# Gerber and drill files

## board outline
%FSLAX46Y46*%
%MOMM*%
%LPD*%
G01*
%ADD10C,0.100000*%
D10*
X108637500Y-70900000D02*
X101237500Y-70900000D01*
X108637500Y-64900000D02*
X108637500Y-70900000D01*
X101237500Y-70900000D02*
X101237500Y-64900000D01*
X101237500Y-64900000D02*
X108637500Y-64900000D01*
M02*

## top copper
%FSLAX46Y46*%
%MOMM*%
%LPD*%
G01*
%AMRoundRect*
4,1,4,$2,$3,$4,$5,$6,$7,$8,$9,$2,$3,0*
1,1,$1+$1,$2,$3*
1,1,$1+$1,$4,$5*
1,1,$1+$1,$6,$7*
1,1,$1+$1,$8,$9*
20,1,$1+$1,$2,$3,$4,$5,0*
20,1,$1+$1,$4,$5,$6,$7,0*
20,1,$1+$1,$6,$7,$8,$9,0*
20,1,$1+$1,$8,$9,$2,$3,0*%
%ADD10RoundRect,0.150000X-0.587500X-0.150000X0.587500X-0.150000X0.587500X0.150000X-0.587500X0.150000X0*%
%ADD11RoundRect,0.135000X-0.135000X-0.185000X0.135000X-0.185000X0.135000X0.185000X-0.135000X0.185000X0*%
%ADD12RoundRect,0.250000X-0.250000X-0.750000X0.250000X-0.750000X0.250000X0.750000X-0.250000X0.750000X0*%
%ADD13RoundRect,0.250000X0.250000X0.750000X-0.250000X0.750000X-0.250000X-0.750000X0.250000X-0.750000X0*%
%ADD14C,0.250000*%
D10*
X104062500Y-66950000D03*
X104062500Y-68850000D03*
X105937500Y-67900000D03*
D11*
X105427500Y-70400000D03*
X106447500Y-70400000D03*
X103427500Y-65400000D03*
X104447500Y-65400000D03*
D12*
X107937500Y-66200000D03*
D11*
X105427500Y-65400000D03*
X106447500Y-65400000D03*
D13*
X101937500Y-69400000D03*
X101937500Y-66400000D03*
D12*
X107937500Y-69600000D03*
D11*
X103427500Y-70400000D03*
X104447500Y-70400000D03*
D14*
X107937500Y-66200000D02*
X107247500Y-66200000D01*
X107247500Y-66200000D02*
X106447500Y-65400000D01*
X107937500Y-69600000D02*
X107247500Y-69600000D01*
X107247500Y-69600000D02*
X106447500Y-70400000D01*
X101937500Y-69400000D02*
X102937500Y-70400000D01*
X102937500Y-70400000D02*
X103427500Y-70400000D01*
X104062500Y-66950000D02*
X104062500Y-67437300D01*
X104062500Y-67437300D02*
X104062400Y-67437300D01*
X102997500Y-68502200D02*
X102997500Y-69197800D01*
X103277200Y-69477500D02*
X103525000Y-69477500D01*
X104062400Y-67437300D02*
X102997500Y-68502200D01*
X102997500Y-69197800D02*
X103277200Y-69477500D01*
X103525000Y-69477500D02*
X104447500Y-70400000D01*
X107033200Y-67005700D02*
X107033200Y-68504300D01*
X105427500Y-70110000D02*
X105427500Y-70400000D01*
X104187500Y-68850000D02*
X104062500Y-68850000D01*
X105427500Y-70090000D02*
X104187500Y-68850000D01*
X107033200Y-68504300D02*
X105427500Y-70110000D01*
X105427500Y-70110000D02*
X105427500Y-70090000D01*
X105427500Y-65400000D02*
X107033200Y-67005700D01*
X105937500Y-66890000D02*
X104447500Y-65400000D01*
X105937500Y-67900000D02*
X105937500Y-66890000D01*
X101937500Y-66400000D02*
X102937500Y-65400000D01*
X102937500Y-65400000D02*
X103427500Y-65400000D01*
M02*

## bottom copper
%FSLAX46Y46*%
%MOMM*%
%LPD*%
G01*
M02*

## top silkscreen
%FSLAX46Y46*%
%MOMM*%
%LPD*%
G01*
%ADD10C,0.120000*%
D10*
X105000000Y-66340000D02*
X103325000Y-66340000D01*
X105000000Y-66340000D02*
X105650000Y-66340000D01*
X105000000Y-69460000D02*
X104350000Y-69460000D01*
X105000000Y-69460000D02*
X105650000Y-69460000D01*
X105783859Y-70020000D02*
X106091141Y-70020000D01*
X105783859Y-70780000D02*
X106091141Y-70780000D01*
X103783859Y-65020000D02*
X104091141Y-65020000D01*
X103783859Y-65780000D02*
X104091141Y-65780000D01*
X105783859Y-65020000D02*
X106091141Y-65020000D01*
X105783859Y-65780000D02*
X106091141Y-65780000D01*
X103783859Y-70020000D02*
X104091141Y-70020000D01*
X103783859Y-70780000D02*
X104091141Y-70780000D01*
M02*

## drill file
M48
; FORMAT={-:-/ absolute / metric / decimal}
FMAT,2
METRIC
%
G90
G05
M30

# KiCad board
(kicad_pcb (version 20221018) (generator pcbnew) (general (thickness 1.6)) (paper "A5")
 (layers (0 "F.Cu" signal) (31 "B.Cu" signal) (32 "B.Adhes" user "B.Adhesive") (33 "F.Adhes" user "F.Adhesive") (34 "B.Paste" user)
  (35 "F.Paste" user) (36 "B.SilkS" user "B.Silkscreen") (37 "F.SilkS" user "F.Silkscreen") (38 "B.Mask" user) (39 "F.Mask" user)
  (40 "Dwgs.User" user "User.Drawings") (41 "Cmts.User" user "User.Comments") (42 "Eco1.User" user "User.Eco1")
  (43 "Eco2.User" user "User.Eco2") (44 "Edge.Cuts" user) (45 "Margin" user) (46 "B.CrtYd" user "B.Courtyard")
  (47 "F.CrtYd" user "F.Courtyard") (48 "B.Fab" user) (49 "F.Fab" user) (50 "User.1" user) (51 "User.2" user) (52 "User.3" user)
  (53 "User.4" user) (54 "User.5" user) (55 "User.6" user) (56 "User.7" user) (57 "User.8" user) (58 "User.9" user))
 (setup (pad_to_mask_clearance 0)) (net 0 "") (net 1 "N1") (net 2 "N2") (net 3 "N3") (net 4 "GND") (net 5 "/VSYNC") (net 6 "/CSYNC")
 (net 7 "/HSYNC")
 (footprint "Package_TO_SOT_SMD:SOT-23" (layer "F.Cu") (at 105 67.9)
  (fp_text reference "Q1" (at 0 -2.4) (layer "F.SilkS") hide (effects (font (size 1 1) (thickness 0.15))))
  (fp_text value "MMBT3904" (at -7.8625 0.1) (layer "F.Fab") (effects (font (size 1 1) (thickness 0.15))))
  (fp_line (start 0 -1.56) (end -1.675 -1.56) (stroke (width 0.12) (type solid)) (layer "F.SilkS"))
  (fp_line (start 0 -1.56) (end 0.65 -1.56) (stroke (width 0.12) (type solid)) (layer "F.SilkS"))
  (fp_line (start 0 1.56) (end -0.65 1.56) (stroke (width 0.12) (type solid)) (layer "F.SilkS"))
  (fp_line (start 0 1.56) (end 0.65 1.56) (stroke (width 0.12) (type solid)) (layer "F.SilkS"))
  (pad "1" smd roundrect (at -0.9375 -0.95) (size 1.475 0.6) (layers "F.Cu" "F.Paste" "F.Mask") (roundrect_rratio 0.25) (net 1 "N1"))
  (pad "2" smd roundrect (at -0.9375 0.95) (size 1.475 0.6) (layers "F.Cu" "F.Paste" "F.Mask") (roundrect_rratio 0.25) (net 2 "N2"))
  (pad "3" smd roundrect (at 0.9375 0) (size 1.475 0.6) (layers "F.Cu" "F.Paste" "F.Mask") (roundrect_rratio 0.25) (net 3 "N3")))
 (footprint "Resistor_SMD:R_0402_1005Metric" (layer "F.Cu") (at 105.9375 70.4)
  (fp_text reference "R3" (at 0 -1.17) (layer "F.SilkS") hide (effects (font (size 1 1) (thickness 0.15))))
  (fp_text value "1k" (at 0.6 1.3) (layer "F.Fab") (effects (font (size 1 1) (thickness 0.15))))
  (fp_line (start -0.153641 -0.38) (end 0.153641 -0.38) (stroke (width 0.12) (type solid)) (layer "F.SilkS"))
  (fp_line (start -0.153641 0.38) (end 0.153641 0.38) (stroke (width 0.12) (type solid)) (layer "F.SilkS"))
  (pad "1" smd roundrect (at -0.51 0) (size 0.54 0.64) (layers "F.Cu" "F.Paste" "F.Mask") (roundrect_rratio 0.25) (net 2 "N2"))
  (pad "2" smd roundrect (at 0.51 0) (size 0.54 0.64) (layers "F.Cu" "F.Paste" "F.Mask") (roundrect_rratio 0.25) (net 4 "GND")))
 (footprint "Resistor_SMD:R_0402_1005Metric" (layer "F.Cu") (at 103.9375 65.4)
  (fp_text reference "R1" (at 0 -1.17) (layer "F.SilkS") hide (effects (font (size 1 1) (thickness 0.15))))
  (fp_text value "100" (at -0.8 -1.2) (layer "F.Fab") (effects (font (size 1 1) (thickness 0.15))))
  (fp_line (start -0.153641 -0.38) (end 0.153641 -0.38) (stroke (width 0.12) (type solid)) (layer "F.SilkS"))
  (fp_line (start -0.153641 0.38) (end 0.153641 0.38) (stroke (width 0.12) (type solid)) (layer "F.SilkS"))
  (pad "1" smd roundrect (at -0.51 0) (size 0.54 0.64) (layers "F.Cu" "F.Paste" "F.Mask") (roundrect_rratio 0.25) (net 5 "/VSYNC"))
  (pad "2" smd roundrect (at 0.51 0) (size 0.54 0.64) (layers "F.Cu" "F.Paste" "F.Mask") (roundrect_rratio 0.25) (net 3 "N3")))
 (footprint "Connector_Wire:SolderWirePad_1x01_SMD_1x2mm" (layer "F.Cu") (at 107.9375 66.2)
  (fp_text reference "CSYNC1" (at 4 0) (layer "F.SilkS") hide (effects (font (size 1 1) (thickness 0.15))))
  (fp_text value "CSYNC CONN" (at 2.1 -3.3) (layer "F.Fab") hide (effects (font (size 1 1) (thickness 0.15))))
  (pad "1" smd roundrect (at 0 0) (size 1 2) (layers "F.Cu" "F.Paste" "F.Mask") (roundrect_rratio 0.25) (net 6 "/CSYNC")))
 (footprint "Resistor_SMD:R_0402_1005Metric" (layer "F.Cu") (at 105.9375 65.4)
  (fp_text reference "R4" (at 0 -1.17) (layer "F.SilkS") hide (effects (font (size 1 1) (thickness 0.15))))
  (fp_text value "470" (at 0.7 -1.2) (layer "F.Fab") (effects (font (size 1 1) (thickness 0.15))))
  (fp_line (start -0.153641 -0.38) (end 0.153641 -0.38) (stroke (width 0.12) (type solid)) (layer "F.SilkS"))
  (fp_line (start -0.153641 0.38) (end 0.153641 0.38) (stroke (width 0.12) (type solid)) (layer "F.SilkS"))
  (pad "1" smd roundrect (at -0.51 0) (size 0.54 0.64) (layers "F.Cu" "F.Paste" "F.Mask") (roundrect_rratio 0.25) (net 2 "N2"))
  (pad "2" smd roundrect (at 0.51 0) (size 0.54 0.64) (layers "F.Cu" "F.Paste" "F.Mask") (roundrect_rratio 0.25) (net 6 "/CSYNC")))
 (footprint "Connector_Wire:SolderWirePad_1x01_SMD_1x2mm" (layer "F.Cu") (at 101.9375 69.4 180)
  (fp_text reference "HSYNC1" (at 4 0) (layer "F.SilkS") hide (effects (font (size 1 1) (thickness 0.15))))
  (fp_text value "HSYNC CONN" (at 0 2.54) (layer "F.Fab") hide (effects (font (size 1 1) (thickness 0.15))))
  (pad "1" smd roundrect (at 0 0 180) (size 1 2) (layers "F.Cu" "F.Paste" "F.Mask") (roundrect_rratio 0.25) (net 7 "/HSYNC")))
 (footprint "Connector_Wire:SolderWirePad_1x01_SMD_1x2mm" (layer "F.Cu") (at 101.9375 66.4 180)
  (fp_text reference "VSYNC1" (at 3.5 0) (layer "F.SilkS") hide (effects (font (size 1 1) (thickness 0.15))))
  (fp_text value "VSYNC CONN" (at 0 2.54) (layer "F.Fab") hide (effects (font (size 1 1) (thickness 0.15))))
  (pad "1" smd roundrect (at 0 0 180) (size 1 2) (layers "F.Cu" "F.Paste" "F.Mask") (roundrect_rratio 0.25) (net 5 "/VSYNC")))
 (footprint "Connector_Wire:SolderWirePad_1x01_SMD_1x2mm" (layer "F.Cu") (at 107.9375 69.6)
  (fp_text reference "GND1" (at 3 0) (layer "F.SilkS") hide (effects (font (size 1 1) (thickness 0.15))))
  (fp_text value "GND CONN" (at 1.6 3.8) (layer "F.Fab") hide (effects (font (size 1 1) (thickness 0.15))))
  (pad "1" smd roundrect (at 0 0) (size 1 2) (layers "F.Cu" "F.Paste" "F.Mask") (roundrect_rratio 0.25) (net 4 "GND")))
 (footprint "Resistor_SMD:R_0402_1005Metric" (layer "F.Cu") (at 103.9375 70.4)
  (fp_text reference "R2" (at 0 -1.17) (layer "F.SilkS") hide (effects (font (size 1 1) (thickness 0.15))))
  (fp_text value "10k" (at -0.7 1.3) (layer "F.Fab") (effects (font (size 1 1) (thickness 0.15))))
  (fp_line (start -0.153641 -0.38) (end 0.153641 -0.38) (stroke (width 0.12) (type solid)) (layer "F.SilkS"))
  (fp_line (start -0.153641 0.38) (end 0.153641 0.38) (stroke (width 0.12) (type solid)) (layer "F.SilkS"))
  (pad "1" smd roundrect (at -0.51 0) (size 0.54 0.64) (layers "F.Cu" "F.Paste" "F.Mask") (roundrect_rratio 0.25) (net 7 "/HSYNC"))
  (pad "2" smd roundrect (at 0.51 0) (size 0.54 0.64) (layers "F.Cu" "F.Paste" "F.Mask") (roundrect_rratio 0.25) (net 1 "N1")))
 (gr_line (start 108.6375 70.9) (end 101.2375 70.9) (stroke (width 0.1) (type default)) (layer "Edge.Cuts"))
 (gr_line (start 108.6375 64.9) (end 108.6375 70.9) (stroke (width 0.1) (type default)) (layer "Edge.Cuts"))
 (gr_line (start 101.2375 70.9) (end 101.2375 64.9) (stroke (width 0.1) (type default)) (layer "Edge.Cuts"))
 (gr_line (start 101.2375 64.9) (end 108.6375 64.9) (stroke (width 0.1) (type default)) (layer "Edge.Cuts"))
 (segment (start 107.9375 66.2) (end 107.2475 66.2) (width 0.25) (layer "F.Cu") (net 6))
 (segment (start 107.2475 66.2) (end 106.4475 65.4) (width 0.25) (layer "F.Cu") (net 6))
 (segment (start 107.9375 69.6) (end 107.2475 69.6) (width 0.25) (layer "F.Cu") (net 4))
 (segment (start 107.2475 69.6) (end 106.4475 70.4) (width 0.25) (layer "F.Cu") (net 4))
 (segment (start 101.9375 69.4) (end 102.9375 70.4) (width 0.25) (layer "F.Cu") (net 7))
 (segment (start 102.9375 70.4) (end 103.4275 70.4) (width 0.25) (layer "F.Cu") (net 7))
 (segment (start 104.0625 66.95) (end 104.0625 67.4373) (width 0.25) (layer "F.Cu") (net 1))
 (segment (start 104.0625 67.4373) (end 104.0624 67.4373) (width 0.25) (layer "F.Cu") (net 1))
 (segment (start 102.9975 68.5022) (end 102.9975 69.1978) (width 0.25) (layer "F.Cu") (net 1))
 (segment (start 103.2772 69.4775) (end 103.525 69.4775) (width 0.25) (layer "F.Cu") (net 1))
 (segment (start 104.0624 67.4373) (end 102.9975 68.5022) (width 0.25) (layer "F.Cu") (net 1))
 (segment (start 102.9975 69.1978) (end 103.2772 69.4775) (width 0.25) (layer "F.Cu") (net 1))
 (segment (start 103.525 69.4775) (end 104.4475 70.4) (width 0.25) (layer "F.Cu") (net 1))
 (segment (start 107.0332 67.0057) (end 107.0332 68.5043) (width 0.25) (layer "F.Cu") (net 2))
 (segment (start 105.4275 70.11) (end 105.4275 70.4) (width 0.25) (layer "F.Cu") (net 2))
 (segment (start 104.1875 68.85) (end 104.0625 68.85) (width 0.25) (layer "F.Cu") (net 2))
 (segment (start 105.4275 70.09) (end 104.1875 68.85) (width 0.25) (layer "F.Cu") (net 2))
 (segment (start 107.0332 68.5043) (end 105.4275 70.11) (width 0.25) (layer "F.Cu") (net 2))
 (segment (start 105.4275 70.11) (end 105.4275 70.09) (width 0.25) (layer "F.Cu") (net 2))
 (segment (start 105.4275 65.4) (end 107.0332 67.0057) (width 0.25) (layer "F.Cu") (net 2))
 (segment (start 105.9375 66.89) (end 104.4475 65.4) (width 0.25) (layer "F.Cu") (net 3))
 (segment (start 105.9375 67.9) (end 105.9375 66.89) (width 0.25) (layer "F.Cu") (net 3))
 (segment (start 101.9375 66.4) (end 102.9375 65.4) (width 0.25) (layer "F.Cu") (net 5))
 (segment (start 102.9375 65.4) (end 103.4275 65.4) (width 0.25) (layer "F.Cu") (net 5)))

